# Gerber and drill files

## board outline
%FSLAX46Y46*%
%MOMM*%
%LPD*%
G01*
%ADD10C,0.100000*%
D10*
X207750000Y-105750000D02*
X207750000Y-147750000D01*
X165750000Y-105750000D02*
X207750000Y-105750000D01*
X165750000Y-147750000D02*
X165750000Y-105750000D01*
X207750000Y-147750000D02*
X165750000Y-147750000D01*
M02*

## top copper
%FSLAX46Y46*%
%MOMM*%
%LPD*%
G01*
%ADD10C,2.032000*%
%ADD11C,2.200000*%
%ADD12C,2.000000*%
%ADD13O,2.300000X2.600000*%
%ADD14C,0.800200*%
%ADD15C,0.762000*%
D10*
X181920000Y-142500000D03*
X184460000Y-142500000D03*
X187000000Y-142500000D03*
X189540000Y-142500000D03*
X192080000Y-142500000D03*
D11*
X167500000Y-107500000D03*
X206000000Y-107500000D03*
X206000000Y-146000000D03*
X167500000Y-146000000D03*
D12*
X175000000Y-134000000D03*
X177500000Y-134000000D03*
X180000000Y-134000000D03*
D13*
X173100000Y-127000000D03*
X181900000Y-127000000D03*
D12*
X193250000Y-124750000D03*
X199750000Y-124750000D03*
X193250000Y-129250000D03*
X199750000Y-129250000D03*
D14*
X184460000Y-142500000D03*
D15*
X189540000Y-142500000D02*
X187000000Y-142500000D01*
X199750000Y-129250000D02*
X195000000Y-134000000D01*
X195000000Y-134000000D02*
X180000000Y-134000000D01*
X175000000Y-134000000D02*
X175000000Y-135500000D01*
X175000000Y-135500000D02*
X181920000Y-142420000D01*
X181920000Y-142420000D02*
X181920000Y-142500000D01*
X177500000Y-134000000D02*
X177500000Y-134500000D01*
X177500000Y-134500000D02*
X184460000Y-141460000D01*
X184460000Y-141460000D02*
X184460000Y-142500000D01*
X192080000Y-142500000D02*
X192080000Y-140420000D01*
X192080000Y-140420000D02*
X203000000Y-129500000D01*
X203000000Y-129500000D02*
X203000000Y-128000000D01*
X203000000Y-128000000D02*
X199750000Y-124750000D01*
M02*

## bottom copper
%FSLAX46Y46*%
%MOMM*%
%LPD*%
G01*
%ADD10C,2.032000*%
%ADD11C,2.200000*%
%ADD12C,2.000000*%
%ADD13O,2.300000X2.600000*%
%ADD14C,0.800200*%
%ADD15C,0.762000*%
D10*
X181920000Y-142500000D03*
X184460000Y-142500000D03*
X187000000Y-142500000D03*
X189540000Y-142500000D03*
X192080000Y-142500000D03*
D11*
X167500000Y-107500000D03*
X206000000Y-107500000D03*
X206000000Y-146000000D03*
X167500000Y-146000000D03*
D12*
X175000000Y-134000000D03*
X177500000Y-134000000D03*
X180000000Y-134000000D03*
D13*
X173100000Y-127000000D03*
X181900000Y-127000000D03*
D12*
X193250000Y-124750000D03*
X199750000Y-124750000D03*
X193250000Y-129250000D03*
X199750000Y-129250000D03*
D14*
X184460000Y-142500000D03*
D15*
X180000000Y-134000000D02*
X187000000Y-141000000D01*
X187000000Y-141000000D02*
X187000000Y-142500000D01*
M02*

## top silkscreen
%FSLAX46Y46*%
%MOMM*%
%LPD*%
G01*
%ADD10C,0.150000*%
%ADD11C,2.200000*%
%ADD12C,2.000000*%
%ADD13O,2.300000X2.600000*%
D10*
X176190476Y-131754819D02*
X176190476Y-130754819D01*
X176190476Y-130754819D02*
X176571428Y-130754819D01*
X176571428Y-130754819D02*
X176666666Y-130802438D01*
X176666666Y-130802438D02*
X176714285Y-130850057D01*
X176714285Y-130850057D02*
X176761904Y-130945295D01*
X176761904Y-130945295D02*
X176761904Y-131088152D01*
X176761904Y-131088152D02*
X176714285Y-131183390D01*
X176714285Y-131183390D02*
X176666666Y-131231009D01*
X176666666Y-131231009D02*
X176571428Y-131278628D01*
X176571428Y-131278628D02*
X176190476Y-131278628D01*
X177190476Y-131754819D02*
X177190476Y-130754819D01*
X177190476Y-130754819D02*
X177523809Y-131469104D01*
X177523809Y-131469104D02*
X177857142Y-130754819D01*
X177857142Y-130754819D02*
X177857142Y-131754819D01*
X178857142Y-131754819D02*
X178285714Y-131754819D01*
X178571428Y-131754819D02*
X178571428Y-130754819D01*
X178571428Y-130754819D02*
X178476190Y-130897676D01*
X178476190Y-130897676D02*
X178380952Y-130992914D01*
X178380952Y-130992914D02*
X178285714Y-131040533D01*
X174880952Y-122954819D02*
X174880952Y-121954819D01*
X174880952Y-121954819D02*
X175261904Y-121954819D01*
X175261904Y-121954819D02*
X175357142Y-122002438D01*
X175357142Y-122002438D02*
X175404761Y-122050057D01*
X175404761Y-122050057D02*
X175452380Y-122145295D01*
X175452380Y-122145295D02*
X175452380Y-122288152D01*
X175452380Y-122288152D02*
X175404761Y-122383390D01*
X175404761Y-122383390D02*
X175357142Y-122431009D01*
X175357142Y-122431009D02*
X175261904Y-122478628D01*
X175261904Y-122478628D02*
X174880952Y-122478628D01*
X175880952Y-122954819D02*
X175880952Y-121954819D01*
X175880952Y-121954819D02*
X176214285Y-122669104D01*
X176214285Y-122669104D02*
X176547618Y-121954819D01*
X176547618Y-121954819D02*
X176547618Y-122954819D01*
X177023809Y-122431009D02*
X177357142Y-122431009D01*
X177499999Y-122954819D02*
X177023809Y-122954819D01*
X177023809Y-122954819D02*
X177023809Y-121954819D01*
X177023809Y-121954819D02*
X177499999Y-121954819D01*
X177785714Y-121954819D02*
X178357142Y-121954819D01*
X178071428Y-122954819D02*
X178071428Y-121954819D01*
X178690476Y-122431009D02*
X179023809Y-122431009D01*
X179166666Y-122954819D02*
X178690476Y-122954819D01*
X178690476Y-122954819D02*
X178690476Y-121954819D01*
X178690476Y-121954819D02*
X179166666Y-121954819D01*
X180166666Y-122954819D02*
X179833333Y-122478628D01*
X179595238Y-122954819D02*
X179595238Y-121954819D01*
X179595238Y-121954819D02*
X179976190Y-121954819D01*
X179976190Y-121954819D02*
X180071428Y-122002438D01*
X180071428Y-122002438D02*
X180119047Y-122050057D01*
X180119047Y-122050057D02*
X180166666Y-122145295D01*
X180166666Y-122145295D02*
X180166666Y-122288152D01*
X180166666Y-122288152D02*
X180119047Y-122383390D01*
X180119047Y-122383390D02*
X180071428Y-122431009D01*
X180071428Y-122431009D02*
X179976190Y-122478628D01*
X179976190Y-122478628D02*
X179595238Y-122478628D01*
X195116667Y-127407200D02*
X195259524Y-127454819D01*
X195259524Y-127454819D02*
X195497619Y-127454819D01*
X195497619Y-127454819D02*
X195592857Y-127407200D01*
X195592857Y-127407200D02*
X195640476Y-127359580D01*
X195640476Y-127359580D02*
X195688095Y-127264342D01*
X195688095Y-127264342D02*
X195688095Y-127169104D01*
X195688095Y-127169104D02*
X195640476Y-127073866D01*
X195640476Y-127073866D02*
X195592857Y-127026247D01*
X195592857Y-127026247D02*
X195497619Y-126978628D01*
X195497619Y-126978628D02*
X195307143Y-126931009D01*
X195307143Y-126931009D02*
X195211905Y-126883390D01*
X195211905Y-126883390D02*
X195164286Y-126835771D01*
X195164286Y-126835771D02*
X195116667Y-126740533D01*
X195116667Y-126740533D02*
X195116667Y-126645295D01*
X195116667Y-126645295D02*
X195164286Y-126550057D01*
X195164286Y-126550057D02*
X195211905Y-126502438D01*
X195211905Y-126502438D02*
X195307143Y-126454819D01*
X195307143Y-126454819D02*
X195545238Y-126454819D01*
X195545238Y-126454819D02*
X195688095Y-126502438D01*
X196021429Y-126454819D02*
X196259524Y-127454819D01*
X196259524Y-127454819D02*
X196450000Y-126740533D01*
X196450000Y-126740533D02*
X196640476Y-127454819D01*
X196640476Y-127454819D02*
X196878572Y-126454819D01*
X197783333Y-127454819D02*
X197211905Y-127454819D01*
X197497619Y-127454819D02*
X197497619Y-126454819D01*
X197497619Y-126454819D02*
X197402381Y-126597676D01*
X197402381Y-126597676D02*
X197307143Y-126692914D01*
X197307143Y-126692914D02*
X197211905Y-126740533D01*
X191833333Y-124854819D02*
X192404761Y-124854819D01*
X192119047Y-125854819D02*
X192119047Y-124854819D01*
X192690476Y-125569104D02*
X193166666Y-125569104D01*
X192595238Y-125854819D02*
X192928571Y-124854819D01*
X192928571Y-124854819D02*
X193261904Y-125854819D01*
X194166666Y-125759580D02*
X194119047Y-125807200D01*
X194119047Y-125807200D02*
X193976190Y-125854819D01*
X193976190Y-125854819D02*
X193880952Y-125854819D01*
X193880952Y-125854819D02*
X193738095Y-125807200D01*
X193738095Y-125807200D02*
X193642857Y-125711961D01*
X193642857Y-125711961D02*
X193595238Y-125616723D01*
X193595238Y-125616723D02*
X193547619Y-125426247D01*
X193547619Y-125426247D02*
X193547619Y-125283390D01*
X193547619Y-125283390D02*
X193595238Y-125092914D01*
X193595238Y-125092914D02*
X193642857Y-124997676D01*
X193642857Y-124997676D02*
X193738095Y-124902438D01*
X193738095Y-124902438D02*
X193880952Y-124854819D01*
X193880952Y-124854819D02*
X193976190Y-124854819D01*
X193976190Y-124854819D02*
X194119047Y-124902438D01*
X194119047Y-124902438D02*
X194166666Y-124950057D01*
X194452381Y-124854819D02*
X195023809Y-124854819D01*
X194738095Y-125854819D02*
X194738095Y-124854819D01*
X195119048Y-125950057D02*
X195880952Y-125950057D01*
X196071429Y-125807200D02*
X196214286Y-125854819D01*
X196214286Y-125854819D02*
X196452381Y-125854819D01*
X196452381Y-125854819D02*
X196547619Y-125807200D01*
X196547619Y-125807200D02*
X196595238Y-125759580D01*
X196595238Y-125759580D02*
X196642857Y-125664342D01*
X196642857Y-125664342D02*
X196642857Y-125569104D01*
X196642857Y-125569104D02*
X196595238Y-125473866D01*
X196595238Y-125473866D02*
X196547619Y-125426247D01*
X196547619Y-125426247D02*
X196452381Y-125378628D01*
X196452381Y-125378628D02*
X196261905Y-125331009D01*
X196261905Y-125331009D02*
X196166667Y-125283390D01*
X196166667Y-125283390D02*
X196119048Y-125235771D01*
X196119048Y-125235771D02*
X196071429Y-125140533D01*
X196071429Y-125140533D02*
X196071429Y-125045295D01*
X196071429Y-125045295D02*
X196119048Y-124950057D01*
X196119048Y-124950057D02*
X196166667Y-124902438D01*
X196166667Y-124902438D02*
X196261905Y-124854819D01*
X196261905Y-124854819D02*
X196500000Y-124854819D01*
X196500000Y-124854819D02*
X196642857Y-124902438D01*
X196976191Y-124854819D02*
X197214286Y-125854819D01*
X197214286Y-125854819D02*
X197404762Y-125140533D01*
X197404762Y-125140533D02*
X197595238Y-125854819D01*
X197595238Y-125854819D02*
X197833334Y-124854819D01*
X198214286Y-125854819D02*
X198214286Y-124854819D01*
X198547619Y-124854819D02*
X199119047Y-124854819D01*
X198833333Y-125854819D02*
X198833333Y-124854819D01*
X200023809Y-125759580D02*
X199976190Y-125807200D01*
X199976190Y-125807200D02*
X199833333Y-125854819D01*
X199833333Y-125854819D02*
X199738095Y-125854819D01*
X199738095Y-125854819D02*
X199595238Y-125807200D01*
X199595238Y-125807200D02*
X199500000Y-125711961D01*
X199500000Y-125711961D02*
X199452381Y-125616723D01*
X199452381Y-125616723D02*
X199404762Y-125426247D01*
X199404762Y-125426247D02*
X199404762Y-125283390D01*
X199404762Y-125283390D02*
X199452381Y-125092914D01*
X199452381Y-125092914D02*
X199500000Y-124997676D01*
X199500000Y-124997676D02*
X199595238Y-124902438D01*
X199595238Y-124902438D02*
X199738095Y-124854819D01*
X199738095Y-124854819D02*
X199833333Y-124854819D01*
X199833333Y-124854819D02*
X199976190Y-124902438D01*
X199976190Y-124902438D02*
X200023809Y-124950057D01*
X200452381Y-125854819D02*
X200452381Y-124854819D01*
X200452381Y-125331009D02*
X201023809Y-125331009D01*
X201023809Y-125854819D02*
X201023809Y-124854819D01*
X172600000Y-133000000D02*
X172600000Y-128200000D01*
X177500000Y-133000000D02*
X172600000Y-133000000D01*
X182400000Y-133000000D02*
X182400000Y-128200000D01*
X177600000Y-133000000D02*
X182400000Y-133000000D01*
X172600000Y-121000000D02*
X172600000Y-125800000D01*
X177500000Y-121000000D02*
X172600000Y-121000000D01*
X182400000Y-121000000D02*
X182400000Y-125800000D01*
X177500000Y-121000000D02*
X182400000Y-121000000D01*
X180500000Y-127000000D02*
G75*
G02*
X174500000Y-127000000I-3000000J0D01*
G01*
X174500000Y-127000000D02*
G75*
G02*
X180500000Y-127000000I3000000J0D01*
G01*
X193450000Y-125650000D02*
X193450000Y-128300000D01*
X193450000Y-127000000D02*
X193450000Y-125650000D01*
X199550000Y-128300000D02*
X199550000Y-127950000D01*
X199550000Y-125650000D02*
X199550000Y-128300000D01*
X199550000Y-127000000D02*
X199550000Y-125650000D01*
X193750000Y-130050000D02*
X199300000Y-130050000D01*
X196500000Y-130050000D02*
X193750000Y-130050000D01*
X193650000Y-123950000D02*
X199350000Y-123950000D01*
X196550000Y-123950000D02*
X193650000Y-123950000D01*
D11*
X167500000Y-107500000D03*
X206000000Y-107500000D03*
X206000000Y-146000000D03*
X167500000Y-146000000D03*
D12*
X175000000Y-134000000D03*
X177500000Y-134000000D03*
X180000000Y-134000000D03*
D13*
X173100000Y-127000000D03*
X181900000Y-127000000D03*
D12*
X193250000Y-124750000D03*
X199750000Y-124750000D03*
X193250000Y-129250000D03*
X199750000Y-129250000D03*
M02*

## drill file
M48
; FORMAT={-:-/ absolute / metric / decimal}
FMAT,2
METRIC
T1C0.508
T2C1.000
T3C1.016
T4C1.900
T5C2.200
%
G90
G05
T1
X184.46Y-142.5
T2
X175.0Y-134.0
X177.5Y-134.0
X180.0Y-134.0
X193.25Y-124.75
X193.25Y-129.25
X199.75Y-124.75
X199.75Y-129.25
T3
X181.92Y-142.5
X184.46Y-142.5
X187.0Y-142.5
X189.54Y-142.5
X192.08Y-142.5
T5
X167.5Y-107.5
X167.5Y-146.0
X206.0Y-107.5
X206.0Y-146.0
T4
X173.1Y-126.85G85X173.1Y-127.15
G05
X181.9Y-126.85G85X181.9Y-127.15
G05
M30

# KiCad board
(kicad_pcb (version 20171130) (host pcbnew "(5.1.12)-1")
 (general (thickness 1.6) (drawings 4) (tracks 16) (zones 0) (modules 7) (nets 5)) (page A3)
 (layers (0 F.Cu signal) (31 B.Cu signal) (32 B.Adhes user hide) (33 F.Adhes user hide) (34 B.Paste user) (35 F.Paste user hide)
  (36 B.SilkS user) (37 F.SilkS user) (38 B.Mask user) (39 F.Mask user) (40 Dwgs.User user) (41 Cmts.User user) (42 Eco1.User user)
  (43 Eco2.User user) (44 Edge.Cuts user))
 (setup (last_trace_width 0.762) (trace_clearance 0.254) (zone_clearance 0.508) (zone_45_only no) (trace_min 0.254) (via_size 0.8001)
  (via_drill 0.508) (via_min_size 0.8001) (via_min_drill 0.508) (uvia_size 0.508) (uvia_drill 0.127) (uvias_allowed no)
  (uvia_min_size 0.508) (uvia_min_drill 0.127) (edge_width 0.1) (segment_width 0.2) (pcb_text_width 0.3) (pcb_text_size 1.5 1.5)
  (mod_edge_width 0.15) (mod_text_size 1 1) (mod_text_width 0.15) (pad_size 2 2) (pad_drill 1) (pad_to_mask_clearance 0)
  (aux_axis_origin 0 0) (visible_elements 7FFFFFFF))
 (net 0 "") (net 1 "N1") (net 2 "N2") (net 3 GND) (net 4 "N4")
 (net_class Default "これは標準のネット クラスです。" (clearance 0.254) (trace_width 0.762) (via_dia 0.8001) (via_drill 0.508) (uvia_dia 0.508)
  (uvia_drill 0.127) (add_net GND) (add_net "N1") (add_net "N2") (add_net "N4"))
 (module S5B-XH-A (layer B.Cu) (at 187 142.5)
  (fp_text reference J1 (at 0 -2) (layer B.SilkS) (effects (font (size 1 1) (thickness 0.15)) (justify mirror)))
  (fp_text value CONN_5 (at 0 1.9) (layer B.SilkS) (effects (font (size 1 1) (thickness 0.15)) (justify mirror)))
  (pad 1 thru_hole circle (at -5.08 0) (size 2.032 2.032) (drill 1.016) (layers *.Cu *.Mask B.SilkS) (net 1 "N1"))
  (pad 2 thru_hole circle (at -2.54 0) (size 2.032 2.032) (drill 1.016) (layers *.Cu *.Mask B.SilkS) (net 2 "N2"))
  (pad 3 thru_hole circle (at 0 0) (size 2.032 2.032) (drill 1.016) (layers *.Cu *.Mask B.SilkS) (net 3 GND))
  (pad 4 thru_hole circle (at 2.54 0) (size 2.032 2.032) (drill 1.016) (layers *.Cu *.Mask B.SilkS) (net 3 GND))
  (pad 5 thru_hole circle (at 5.08 0) (size 2.032 2.032) (drill 1.016) (layers *.Cu *.Mask B.SilkS) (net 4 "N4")))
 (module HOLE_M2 (layer F.Cu) (at 167.5 107.5)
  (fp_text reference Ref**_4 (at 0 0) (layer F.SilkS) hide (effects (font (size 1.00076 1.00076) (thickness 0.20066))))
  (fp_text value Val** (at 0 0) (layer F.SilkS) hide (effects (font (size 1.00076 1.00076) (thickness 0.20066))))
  (pad "" thru_hole circle (at 0 0) (size 2.2 2.2) (drill 2.2) (layers *.Cu *.Mask F.SilkS) (clearance 1.50114)))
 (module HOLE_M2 (layer F.Cu) (at 206 107.5)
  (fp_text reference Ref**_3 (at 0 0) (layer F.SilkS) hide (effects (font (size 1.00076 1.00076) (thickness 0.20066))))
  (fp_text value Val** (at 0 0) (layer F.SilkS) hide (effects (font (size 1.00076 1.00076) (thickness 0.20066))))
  (pad "" thru_hole circle (at 0 0) (size 2.2 2.2) (drill 2.2) (layers *.Cu *.Mask F.SilkS) (clearance 1.50114)))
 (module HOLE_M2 (layer F.Cu) (at 206 146)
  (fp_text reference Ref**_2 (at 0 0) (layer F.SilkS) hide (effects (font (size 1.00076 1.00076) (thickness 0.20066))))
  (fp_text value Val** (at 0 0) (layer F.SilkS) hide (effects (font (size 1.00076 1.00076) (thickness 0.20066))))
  (pad "" thru_hole circle (at 0 0) (size 2.2 2.2) (drill 2.2) (layers *.Cu *.Mask F.SilkS) (clearance 1.50114)))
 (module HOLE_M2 (layer F.Cu) (at 167.5 146)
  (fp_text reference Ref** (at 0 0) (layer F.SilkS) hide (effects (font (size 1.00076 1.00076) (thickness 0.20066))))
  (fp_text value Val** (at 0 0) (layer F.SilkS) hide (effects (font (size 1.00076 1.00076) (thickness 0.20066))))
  (pad "" thru_hole circle (at 0 0) (size 2.2 2.2) (drill 2.2) (layers *.Cu *.Mask F.SilkS) (clearance 1.50114)))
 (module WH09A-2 (layer F.Cu) (at 177.5 127)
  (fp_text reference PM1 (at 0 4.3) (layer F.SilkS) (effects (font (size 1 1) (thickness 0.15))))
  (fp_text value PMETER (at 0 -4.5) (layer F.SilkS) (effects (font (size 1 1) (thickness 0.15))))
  (fp_line (start -4.9 6) (end -4.9 1.2) (layer F.SilkS) (width 0.15))
  (fp_line (start 0 6) (end -4.9 6) (layer F.SilkS) (width 0.15))
  (fp_line (start 4.9 6) (end 4.9 1.2) (layer F.SilkS) (width 0.15))
  (fp_line (start 0.1 6) (end 4.9 6) (layer F.SilkS) (width 0.15))
  (fp_line (start -4.9 -6) (end -4.9 -1.2) (layer F.SilkS) (width 0.15))
  (fp_line (start 0 -6) (end -4.9 -6) (layer F.SilkS) (width 0.15))
  (fp_line (start 4.9 -6) (end 4.9 -1.2) (layer F.SilkS) (width 0.15))
  (fp_line (start 0 -6) (end 4.9 -6) (layer F.SilkS) (width 0.15))
  (fp_circle (center 0 0) (end 0 3) (layer F.SilkS) (width 0.15))
  (pad 1 thru_hole circle (at -2.5 7) (size 2 2) (drill 1) (layers *.Cu *.Mask F.SilkS) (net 1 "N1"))
  (pad 2 thru_hole circle (at 0 7) (size 2 2) (drill 1) (layers *.Cu *.Mask F.SilkS) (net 2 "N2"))
  (pad 3 thru_hole circle (at 2.5 7) (size 2 2) (drill 1) (layers *.Cu *.Mask F.SilkS) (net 3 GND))
  (pad "" thru_hole oval (at -4.4 0) (size 2.3 2.6) (drill oval 1.9 2.2) (layers *.Cu *.Mask F.SilkS))
  (pad "" thru_hole oval (at 4.4 0) (size 2.3 2.6) (drill oval 1.9 2.2) (layers *.Cu *.Mask F.SilkS)))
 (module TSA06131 (layer F.Cu) (at 196.5 127)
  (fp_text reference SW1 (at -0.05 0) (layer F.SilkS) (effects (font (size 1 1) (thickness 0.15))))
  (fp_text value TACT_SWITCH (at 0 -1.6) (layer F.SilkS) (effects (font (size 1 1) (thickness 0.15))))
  (fp_line (start -3.05 -1.35) (end -3.05 1.3) (layer F.SilkS) (width 0.15))
  (fp_line (start -3.05 0) (end -3.05 -1.35) (layer F.SilkS) (width 0.15))
  (fp_line (start 3.05 1.3) (end 3.05 0.95) (layer F.SilkS) (width 0.15))
  (fp_line (start 3.05 -1.35) (end 3.05 1.3) (layer F.SilkS) (width 0.15))
  (fp_line (start 3.05 0) (end 3.05 -1.35) (layer F.SilkS) (width 0.15))
  (fp_line (start -2.75 3.05) (end 2.8 3.05) (layer F.SilkS) (width 0.15))
  (fp_line (start 0 3.05) (end -2.75 3.05) (layer F.SilkS) (width 0.15))
  (fp_line (start -2.85 -3.05) (end 2.85 -3.05) (layer F.SilkS) (width 0.15))
  (fp_line (start 0.05 -3.05) (end -2.85 -3.05) (layer F.SilkS) (width 0.15))
  (pad 4 thru_hole circle (at -3.25 -2.25) (size 2 2) (drill 1) (layers *.Cu *.Mask F.SilkS))
  (pad 1 thru_hole circle (at 3.25 -2.25) (size 2 2) (drill 1) (layers *.Cu *.Mask F.SilkS) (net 4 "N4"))
  (pad 3 thru_hole circle (at -3.25 2.25) (size 2 2) (drill 1) (layers *.Cu *.Mask F.SilkS))
  (pad 2 thru_hole circle (at 3.25 2.25) (size 2 2) (drill 1) (layers *.Cu *.Mask F.SilkS) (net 3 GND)))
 (gr_line (start 207.75 105.75) (end 207.75 147.75) (angle 90) (layer Edge.Cuts) (width 0.1))
 (gr_line (start 165.75 105.75) (end 207.75 105.75) (angle 90) (layer Edge.Cuts) (width 0.1))
 (gr_line (start 165.75 147.75) (end 165.75 105.75) (angle 90) (layer Edge.Cuts) (width 0.1))
 (gr_line (start 207.75 147.75) (end 165.75 147.75) (angle 90) (layer Edge.Cuts) (width 0.1))
 (segment (start 189.54 142.5) (end 187 142.5) (width 0.762) (layer F.Cu) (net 3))
 (segment (start 180 134) (end 187 141) (width 0.762) (layer B.Cu) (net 3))
 (segment (start 187 141) (end 187 142.5) (width 0.762) (layer B.Cu) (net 3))
 (segment (start 199.75 129.25) (end 195 134) (width 0.762) (layer F.Cu) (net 3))
 (segment (start 195 134) (end 180 134) (width 0.762) (layer F.Cu) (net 3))
 (segment (start 175 134) (end 175 135.5) (width 0.762) (layer F.Cu) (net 1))
 (segment (start 175 135.5) (end 181.92 142.42) (width 0.762) (layer F.Cu) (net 1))
 (segment (start 181.92 142.42) (end 181.92 142.5) (width 0.762) (layer F.Cu) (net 1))
 (segment (start 177.5 134) (end 177.5 134.5) (width 0.762) (layer F.Cu) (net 2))
 (segment (start 177.5 134.5) (end 184.46 141.46) (width 0.762) (layer F.Cu) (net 2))
 (segment (start 184.46 141.46) (end 184.46 142.5) (width 0.762) (layer F.Cu) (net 2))
 (via (at 184.46 142.5) (size 0.8002) (layers F.Cu B.Cu) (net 2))
 (segment (start 192.08 142.5) (end 192.08 140.42) (width 0.762) (layer F.Cu) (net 4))
 (segment (start 192.08 140.42) (end 203 129.5) (width 0.762) (layer F.Cu) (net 4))
 (segment (start 203 129.5) (end 203 128) (width 0.762) (layer F.Cu) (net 4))
 (segment (start 203 128) (end 199.75 124.75) (width 0.762) (layer F.Cu) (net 4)))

